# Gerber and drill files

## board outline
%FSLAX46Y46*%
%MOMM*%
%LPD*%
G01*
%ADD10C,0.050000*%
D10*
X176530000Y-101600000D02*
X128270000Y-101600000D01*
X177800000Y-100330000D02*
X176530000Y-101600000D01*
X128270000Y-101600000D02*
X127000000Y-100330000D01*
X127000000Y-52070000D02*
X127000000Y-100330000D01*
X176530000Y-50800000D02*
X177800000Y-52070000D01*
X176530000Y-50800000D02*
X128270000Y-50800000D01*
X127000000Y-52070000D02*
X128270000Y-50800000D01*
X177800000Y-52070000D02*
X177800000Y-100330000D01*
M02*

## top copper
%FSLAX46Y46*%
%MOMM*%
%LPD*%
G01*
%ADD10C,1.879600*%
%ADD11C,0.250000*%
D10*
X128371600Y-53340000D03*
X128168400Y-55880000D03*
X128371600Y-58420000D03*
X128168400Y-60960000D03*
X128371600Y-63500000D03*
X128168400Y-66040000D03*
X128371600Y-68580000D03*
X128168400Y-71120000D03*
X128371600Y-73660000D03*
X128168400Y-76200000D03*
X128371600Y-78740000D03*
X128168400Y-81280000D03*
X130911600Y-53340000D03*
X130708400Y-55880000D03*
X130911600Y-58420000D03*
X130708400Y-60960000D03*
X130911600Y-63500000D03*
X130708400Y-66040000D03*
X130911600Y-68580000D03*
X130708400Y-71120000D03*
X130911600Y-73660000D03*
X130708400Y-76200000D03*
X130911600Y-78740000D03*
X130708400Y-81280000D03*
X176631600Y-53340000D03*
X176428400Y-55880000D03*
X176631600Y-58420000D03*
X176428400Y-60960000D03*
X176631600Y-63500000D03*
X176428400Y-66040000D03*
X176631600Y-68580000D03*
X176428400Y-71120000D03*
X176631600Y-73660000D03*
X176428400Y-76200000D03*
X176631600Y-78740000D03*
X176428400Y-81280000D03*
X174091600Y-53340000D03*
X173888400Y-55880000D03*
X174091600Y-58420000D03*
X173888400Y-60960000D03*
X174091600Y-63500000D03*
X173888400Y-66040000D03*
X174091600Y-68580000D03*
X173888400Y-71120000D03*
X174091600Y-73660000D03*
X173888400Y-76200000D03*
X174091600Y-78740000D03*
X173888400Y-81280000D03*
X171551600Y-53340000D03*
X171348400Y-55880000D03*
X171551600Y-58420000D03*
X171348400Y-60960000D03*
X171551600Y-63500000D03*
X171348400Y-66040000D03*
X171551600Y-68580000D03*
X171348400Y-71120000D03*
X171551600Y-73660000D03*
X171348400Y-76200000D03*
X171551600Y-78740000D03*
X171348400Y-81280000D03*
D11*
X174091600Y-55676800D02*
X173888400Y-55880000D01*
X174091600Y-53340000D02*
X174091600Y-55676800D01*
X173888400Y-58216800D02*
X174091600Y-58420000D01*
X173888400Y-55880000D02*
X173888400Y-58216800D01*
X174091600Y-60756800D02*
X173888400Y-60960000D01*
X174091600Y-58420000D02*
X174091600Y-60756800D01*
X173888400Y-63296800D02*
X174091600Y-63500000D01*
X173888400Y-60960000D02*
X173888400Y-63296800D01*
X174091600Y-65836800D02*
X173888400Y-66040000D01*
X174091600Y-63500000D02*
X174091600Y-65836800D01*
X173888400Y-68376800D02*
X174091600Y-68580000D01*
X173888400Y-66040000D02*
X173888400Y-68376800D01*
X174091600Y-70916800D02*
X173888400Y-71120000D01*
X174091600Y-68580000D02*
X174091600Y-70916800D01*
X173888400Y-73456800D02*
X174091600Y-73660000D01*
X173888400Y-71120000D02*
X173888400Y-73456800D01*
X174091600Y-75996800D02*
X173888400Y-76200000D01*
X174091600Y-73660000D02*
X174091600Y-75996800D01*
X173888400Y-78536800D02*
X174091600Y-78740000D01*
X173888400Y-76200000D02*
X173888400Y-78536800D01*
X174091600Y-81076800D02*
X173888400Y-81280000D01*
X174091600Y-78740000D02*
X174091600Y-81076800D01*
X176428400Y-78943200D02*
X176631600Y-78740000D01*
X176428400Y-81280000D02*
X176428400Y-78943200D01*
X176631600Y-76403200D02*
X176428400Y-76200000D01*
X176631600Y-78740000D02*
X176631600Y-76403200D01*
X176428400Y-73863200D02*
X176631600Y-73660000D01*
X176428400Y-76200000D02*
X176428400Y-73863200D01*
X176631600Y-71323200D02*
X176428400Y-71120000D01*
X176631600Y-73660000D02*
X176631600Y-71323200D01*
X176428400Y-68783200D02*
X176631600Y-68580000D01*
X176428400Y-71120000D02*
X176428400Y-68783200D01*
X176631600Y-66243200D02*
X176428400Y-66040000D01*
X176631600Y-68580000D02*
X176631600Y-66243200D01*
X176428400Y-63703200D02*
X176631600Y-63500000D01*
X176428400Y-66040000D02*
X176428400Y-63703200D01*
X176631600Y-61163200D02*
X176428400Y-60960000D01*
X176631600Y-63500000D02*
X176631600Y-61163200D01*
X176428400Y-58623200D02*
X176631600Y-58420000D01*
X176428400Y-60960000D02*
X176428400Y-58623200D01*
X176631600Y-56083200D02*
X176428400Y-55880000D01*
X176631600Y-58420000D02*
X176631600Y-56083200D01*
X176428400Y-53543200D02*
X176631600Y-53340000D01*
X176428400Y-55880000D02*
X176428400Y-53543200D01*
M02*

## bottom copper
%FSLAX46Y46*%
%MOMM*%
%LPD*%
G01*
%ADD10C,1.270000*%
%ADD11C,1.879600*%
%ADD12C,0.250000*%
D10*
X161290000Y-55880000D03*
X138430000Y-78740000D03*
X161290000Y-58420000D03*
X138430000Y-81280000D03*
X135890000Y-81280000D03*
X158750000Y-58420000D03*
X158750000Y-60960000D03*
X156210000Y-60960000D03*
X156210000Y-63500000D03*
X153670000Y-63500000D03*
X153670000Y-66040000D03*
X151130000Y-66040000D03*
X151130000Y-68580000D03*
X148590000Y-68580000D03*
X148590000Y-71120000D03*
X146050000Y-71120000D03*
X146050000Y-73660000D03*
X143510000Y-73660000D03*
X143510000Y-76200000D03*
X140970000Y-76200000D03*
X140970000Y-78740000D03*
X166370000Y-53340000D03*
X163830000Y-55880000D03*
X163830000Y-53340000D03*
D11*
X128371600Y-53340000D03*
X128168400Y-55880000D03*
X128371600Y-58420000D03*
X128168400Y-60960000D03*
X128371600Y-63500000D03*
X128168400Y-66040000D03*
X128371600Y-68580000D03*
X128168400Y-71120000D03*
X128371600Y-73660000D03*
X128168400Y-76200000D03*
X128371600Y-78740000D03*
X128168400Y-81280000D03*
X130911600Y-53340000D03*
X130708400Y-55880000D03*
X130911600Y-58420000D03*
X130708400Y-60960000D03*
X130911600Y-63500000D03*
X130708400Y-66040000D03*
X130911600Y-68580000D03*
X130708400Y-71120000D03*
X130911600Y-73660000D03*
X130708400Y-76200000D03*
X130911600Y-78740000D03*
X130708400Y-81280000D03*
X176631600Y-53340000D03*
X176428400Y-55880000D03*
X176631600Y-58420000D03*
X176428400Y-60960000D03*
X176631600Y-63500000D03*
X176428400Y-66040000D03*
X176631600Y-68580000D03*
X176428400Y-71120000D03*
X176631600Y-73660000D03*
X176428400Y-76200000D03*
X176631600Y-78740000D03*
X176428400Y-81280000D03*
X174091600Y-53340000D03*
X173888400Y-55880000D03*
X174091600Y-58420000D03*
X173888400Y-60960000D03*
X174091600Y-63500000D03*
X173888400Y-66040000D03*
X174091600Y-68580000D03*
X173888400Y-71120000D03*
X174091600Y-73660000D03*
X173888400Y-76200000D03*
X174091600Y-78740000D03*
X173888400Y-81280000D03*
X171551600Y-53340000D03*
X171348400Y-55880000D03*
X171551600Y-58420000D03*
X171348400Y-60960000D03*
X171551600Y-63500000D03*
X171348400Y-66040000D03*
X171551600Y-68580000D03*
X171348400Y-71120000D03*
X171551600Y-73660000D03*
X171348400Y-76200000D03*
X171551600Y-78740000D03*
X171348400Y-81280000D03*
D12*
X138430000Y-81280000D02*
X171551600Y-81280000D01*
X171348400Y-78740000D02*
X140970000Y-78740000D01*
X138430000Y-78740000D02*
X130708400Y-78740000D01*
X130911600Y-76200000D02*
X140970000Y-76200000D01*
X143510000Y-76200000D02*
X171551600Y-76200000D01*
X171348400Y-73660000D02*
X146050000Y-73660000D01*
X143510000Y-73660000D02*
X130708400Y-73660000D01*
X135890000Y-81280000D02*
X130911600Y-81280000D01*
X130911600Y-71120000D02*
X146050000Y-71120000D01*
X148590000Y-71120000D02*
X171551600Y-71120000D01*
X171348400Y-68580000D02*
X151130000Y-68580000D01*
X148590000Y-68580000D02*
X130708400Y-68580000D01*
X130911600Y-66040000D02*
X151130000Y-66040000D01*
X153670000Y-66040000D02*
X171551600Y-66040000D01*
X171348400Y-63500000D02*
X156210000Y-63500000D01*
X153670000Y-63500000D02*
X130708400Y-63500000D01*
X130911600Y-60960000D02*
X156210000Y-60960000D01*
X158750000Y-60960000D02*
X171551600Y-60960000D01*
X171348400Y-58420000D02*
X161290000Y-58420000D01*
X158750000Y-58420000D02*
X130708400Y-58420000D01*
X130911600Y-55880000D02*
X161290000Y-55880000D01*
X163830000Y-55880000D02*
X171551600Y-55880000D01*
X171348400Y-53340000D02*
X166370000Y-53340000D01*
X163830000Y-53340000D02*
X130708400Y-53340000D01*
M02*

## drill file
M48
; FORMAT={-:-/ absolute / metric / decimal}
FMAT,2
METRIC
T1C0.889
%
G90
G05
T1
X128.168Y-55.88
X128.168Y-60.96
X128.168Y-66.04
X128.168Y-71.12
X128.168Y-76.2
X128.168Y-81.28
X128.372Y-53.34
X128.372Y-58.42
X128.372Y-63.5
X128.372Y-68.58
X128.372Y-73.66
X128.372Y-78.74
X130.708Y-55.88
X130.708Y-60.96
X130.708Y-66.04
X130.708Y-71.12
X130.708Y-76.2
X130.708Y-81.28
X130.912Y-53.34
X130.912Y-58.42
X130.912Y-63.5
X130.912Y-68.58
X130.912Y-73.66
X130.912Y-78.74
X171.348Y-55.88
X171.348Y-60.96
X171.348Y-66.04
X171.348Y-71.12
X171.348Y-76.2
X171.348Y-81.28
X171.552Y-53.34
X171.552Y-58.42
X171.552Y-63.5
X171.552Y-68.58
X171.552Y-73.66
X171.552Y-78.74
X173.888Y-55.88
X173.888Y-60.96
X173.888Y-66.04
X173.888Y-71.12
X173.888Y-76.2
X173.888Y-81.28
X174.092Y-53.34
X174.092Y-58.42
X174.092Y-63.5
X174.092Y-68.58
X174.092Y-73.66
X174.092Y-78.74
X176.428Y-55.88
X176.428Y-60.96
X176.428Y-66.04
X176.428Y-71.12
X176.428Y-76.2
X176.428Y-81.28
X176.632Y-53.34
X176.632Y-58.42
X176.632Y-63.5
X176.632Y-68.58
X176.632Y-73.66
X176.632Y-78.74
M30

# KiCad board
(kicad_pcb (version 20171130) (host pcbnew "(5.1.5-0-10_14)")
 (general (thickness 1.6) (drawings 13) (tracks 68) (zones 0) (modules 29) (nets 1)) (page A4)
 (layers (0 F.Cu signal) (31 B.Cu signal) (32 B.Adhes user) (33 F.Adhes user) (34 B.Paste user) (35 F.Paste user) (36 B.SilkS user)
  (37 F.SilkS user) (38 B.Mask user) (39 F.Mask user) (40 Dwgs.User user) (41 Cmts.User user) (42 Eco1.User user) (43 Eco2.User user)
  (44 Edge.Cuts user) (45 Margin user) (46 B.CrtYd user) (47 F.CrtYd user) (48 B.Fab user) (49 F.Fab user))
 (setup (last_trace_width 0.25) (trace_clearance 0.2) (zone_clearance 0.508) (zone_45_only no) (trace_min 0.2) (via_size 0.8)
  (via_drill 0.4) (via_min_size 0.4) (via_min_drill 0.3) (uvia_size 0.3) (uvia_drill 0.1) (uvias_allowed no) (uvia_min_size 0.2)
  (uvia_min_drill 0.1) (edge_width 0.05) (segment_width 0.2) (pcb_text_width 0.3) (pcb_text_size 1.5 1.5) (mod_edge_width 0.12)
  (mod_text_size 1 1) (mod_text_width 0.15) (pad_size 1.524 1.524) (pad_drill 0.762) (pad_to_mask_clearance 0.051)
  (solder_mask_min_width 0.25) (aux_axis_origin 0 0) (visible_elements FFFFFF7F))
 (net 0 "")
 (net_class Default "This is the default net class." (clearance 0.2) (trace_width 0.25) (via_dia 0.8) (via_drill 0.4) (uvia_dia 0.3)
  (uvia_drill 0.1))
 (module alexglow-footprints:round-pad (layer B.Cu) (at 161.29 55.88)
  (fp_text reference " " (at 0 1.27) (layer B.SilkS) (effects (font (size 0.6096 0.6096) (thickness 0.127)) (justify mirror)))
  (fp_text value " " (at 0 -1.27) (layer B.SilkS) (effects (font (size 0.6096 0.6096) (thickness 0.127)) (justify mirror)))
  (pad P$1 smd circle (at 0 0) (size 1.27 1.27) (layers B.Cu B.Paste B.Mask) (solder_mask_margin 0.1016)))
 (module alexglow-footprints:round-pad (layer B.Cu) (at 138.43 78.74)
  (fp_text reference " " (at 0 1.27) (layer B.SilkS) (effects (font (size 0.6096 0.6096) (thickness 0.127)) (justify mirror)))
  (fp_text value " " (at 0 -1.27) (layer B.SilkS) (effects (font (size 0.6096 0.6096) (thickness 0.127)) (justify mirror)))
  (pad P$1 smd circle (at 0 0) (size 1.27 1.27) (layers B.Cu B.Paste B.Mask) (solder_mask_margin 0.1016)))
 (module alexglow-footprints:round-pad (layer B.Cu) (at 161.29 58.42)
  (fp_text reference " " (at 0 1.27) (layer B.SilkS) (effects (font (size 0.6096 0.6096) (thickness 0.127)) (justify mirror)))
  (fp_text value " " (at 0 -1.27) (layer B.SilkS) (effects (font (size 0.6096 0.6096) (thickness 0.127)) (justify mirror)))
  (pad P$1 smd circle (at 0 0) (size 1.27 1.27) (layers B.Cu B.Paste B.Mask) (solder_mask_margin 0.1016)))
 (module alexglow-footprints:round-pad (layer B.Cu) (at 138.43 81.28)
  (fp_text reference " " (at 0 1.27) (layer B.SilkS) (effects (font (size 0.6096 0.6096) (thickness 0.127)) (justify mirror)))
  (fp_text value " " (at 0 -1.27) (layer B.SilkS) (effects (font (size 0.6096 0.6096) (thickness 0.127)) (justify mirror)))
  (pad P$1 smd circle (at 0 0) (size 1.27 1.27) (layers B.Cu B.Paste B.Mask) (solder_mask_margin 0.1016)))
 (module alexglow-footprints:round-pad (layer B.Cu) (at 135.89 81.28)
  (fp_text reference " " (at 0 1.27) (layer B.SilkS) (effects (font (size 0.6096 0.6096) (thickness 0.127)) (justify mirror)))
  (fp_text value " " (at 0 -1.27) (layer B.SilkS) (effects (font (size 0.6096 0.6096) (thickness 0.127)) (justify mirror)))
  (pad P$1 smd circle (at 0 0) (size 1.27 1.27) (layers B.Cu B.Paste B.Mask) (solder_mask_margin 0.1016)))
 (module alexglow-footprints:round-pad (layer B.Cu) (at 158.75 58.42)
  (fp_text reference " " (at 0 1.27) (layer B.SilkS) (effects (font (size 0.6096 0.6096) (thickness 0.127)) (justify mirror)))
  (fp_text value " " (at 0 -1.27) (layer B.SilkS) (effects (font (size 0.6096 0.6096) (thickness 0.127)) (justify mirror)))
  (pad P$1 smd circle (at 0 0) (size 1.27 1.27) (layers B.Cu B.Paste B.Mask) (solder_mask_margin 0.1016)))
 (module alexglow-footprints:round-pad (layer B.Cu) (at 158.75 60.96)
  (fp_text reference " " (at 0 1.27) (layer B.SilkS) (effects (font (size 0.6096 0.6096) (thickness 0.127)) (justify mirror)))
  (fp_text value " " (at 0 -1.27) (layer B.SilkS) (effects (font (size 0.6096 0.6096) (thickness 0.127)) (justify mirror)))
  (pad P$1 smd circle (at 0 0) (size 1.27 1.27) (layers B.Cu B.Paste B.Mask) (solder_mask_margin 0.1016)))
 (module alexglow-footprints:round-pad (layer B.Cu) (at 156.21 60.96)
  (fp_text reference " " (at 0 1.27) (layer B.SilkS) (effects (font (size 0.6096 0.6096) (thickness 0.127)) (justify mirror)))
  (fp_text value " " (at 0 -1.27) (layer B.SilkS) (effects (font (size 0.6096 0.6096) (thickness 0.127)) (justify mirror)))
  (pad P$1 smd circle (at 0 0) (size 1.27 1.27) (layers B.Cu B.Paste B.Mask) (solder_mask_margin 0.1016)))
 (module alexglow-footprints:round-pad (layer B.Cu) (at 156.21 63.5)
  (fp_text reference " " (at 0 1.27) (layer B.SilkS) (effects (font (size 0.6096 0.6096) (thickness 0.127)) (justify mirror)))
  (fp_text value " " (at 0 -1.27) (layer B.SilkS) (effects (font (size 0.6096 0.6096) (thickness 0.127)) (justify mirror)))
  (pad P$1 smd circle (at 0 0) (size 1.27 1.27) (layers B.Cu B.Paste B.Mask) (solder_mask_margin 0.1016)))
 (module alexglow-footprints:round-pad (layer B.Cu) (at 153.67 63.5)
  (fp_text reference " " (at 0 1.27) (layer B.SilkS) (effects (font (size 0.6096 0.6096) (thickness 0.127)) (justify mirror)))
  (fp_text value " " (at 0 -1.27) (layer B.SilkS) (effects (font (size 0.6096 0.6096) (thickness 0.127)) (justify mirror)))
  (pad P$1 smd circle (at 0 0) (size 1.27 1.27) (layers B.Cu B.Paste B.Mask) (solder_mask_margin 0.1016)))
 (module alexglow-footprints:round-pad (layer B.Cu) (at 153.67 66.04)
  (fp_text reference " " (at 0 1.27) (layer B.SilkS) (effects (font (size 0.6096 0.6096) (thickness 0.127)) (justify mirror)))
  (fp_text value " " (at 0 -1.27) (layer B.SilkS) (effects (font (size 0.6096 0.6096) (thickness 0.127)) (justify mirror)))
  (pad P$1 smd circle (at 0 0) (size 1.27 1.27) (layers B.Cu B.Paste B.Mask) (solder_mask_margin 0.1016)))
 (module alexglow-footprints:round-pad (layer B.Cu) (at 151.13 66.04)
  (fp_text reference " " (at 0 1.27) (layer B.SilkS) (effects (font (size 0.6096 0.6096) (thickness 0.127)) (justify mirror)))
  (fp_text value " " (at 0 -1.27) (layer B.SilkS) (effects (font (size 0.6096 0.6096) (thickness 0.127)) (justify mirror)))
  (pad P$1 smd circle (at 0 0) (size 1.27 1.27) (layers B.Cu B.Paste B.Mask) (solder_mask_margin 0.1016)))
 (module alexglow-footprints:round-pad (layer B.Cu) (at 151.13 68.58)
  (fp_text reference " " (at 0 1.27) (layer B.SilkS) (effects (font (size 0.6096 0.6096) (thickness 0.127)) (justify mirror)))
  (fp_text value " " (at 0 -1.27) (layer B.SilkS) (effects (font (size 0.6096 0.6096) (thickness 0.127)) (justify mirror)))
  (pad P$1 smd circle (at 0 0) (size 1.27 1.27) (layers B.Cu B.Paste B.Mask) (solder_mask_margin 0.1016)))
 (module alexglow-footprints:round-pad (layer B.Cu) (at 148.59 68.58)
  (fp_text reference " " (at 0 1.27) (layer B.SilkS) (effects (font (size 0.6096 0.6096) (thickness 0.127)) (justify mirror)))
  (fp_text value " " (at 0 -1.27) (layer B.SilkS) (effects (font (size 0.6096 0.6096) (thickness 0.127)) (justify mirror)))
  (pad P$1 smd circle (at 0 0) (size 1.27 1.27) (layers B.Cu B.Paste B.Mask) (solder_mask_margin 0.1016)))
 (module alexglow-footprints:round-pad (layer B.Cu) (at 148.59 71.12)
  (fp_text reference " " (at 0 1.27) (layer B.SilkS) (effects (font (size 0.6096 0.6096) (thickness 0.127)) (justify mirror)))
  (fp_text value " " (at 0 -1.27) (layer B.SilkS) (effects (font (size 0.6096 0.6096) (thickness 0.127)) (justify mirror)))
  (pad P$1 smd circle (at 0 0) (size 1.27 1.27) (layers B.Cu B.Paste B.Mask) (solder_mask_margin 0.1016)))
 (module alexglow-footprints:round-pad (layer B.Cu) (at 146.05 71.12)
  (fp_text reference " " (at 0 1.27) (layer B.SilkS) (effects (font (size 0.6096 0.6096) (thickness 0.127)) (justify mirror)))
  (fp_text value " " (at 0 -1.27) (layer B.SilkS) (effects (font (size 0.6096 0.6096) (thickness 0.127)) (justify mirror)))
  (pad P$1 smd circle (at 0 0) (size 1.27 1.27) (layers B.Cu B.Paste B.Mask) (solder_mask_margin 0.1016)))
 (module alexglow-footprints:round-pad (layer B.Cu) (at 146.05 73.66)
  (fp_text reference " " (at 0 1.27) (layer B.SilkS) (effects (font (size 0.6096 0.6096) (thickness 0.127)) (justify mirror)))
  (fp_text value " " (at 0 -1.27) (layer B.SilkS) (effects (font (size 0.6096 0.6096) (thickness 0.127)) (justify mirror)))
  (pad P$1 smd circle (at 0 0) (size 1.27 1.27) (layers B.Cu B.Paste B.Mask) (solder_mask_margin 0.1016)))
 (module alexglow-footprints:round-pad (layer B.Cu) (at 143.51 73.66)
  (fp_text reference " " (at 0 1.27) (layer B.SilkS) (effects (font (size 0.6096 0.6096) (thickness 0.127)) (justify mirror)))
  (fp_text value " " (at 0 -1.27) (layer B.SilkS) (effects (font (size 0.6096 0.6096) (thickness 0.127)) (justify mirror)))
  (pad P$1 smd circle (at 0 0) (size 1.27 1.27) (layers B.Cu B.Paste B.Mask) (solder_mask_margin 0.1016)))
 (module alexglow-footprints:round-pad (layer B.Cu) (at 143.51 76.2)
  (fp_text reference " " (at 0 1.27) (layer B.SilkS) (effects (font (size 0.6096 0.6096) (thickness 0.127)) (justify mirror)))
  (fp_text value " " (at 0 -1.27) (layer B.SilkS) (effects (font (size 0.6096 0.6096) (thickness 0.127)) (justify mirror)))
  (pad P$1 smd circle (at 0 0) (size 1.27 1.27) (layers B.Cu B.Paste B.Mask) (solder_mask_margin 0.1016)))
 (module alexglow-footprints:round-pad (layer B.Cu) (at 140.97 76.2)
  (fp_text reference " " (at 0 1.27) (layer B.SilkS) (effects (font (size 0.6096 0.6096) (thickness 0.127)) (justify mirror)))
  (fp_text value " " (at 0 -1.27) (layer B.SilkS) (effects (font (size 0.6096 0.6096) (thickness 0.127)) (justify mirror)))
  (pad P$1 smd circle (at 0 0) (size 1.27 1.27) (layers B.Cu B.Paste B.Mask) (solder_mask_margin 0.1016)))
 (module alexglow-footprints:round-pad (layer B.Cu) (at 140.97 78.74)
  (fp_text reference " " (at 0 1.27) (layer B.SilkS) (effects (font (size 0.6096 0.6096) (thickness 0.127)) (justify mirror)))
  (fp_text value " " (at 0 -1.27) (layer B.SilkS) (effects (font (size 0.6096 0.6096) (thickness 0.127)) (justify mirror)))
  (pad P$1 smd circle (at 0 0) (size 1.27 1.27) (layers B.Cu B.Paste B.Mask) (solder_mask_margin 0.1016)))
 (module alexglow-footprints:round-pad (layer B.Cu) (at 166.37 53.34)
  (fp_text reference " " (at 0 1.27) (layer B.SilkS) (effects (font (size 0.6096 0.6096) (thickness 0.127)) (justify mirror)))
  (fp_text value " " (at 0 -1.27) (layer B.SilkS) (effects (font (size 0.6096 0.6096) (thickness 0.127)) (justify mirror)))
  (pad P$1 smd circle (at 0 0) (size 1.27 1.27) (layers B.Cu B.Paste B.Mask) (solder_mask_margin 0.1016)))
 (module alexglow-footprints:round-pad (layer B.Cu) (at 163.83 55.88)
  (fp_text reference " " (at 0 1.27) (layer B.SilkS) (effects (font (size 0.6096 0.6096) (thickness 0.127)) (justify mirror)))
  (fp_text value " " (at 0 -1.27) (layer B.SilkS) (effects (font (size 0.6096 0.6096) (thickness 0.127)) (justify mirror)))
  (pad P$1 smd circle (at 0 0) (size 1.27 1.27) (layers B.Cu B.Paste B.Mask) (solder_mask_margin 0.1016)))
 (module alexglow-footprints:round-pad (layer B.Cu) (at 163.83 53.34)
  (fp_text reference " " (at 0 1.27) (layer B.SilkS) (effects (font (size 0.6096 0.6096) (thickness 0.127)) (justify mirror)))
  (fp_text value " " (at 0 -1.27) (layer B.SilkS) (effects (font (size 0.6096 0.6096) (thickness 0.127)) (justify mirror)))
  (pad P$1 smd circle (at 0 0) (size 1.27 1.27) (layers B.Cu B.Paste B.Mask) (solder_mask_margin 0.1016)))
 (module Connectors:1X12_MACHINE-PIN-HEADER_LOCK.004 (layer F.Cu) (at 128.27 81.28 90)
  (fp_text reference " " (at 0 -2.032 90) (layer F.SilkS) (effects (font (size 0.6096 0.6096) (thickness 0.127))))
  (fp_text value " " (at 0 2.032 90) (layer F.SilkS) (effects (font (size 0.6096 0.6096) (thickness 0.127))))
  (pad 12 thru_hole circle (at 27.94 0.1016 90) (size 1.8796 1.8796) (drill 0.889) (layers *.Cu *.Mask) (solder_mask_margin 0.1016))
  (pad 11 thru_hole circle (at 25.4 -0.1016 90) (size 1.8796 1.8796) (drill 0.889) (layers *.Cu *.Mask) (solder_mask_margin 0.1016))
  (pad 10 thru_hole circle (at 22.86 0.1016 90) (size 1.8796 1.8796) (drill 0.889) (layers *.Cu *.Mask) (solder_mask_margin 0.1016))
  (pad 9 thru_hole circle (at 20.32 -0.1016 90) (size 1.8796 1.8796) (drill 0.889) (layers *.Cu *.Mask) (solder_mask_margin 0.1016))
  (pad 8 thru_hole circle (at 17.78 0.1016 90) (size 1.8796 1.8796) (drill 0.889) (layers *.Cu *.Mask) (solder_mask_margin 0.1016))
  (pad 7 thru_hole circle (at 15.24 -0.1016 90) (size 1.8796 1.8796) (drill 0.889) (layers *.Cu *.Mask) (solder_mask_margin 0.1016))
  (pad 6 thru_hole circle (at 12.7 0.1016 90) (size 1.8796 1.8796) (drill 0.889) (layers *.Cu *.Mask) (solder_mask_margin 0.1016))
  (pad 5 thru_hole circle (at 10.16 -0.1016 90) (size 1.8796 1.8796) (drill 0.889) (layers *.Cu *.Mask) (solder_mask_margin 0.1016))
  (pad 4 thru_hole circle (at 7.62 0.1016 90) (size 1.8796 1.8796) (drill 0.889) (layers *.Cu *.Mask) (solder_mask_margin 0.1016))
  (pad 3 thru_hole circle (at 5.08 -0.1016 90) (size 1.8796 1.8796) (drill 0.889) (layers *.Cu *.Mask) (solder_mask_margin 0.1016))
  (pad 2 thru_hole circle (at 2.54 0.1016 90) (size 1.8796 1.8796) (drill 0.889) (layers *.Cu *.Mask) (solder_mask_margin 0.1016))
  (pad 1 thru_hole circle (at 0 -0.1016 90) (size 1.8796 1.8796) (drill 0.889) (layers *.Cu *.Mask) (solder_mask_margin 0.1016)))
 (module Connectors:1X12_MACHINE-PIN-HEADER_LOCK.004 (layer F.Cu) (at 130.81 81.28 90)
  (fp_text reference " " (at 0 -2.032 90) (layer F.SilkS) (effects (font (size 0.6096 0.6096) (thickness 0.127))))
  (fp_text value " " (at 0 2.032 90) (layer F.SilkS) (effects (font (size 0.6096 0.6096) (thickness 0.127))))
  (pad 12 thru_hole circle (at 27.94 0.1016 90) (size 1.8796 1.8796) (drill 0.889) (layers *.Cu *.Mask) (solder_mask_margin 0.1016))
  (pad 11 thru_hole circle (at 25.4 -0.1016 90) (size 1.8796 1.8796) (drill 0.889) (layers *.Cu *.Mask) (solder_mask_margin 0.1016))
  (pad 10 thru_hole circle (at 22.86 0.1016 90) (size 1.8796 1.8796) (drill 0.889) (layers *.Cu *.Mask) (solder_mask_margin 0.1016))
  (pad 9 thru_hole circle (at 20.32 -0.1016 90) (size 1.8796 1.8796) (drill 0.889) (layers *.Cu *.Mask) (solder_mask_margin 0.1016))
  (pad 8 thru_hole circle (at 17.78 0.1016 90) (size 1.8796 1.8796) (drill 0.889) (layers *.Cu *.Mask) (solder_mask_margin 0.1016))
  (pad 7 thru_hole circle (at 15.24 -0.1016 90) (size 1.8796 1.8796) (drill 0.889) (layers *.Cu *.Mask) (solder_mask_margin 0.1016))
  (pad 6 thru_hole circle (at 12.7 0.1016 90) (size 1.8796 1.8796) (drill 0.889) (layers *.Cu *.Mask) (solder_mask_margin 0.1016))
  (pad 5 thru_hole circle (at 10.16 -0.1016 90) (size 1.8796 1.8796) (drill 0.889) (layers *.Cu *.Mask) (solder_mask_margin 0.1016))
  (pad 4 thru_hole circle (at 7.62 0.1016 90) (size 1.8796 1.8796) (drill 0.889) (layers *.Cu *.Mask) (solder_mask_margin 0.1016))
  (pad 3 thru_hole circle (at 5.08 -0.1016 90) (size 1.8796 1.8796) (drill 0.889) (layers *.Cu *.Mask) (solder_mask_margin 0.1016))
  (pad 2 thru_hole circle (at 2.54 0.1016 90) (size 1.8796 1.8796) (drill 0.889) (layers *.Cu *.Mask) (solder_mask_margin 0.1016))
  (pad 1 thru_hole circle (at 0 -0.1016 90) (size 1.8796 1.8796) (drill 0.889) (layers *.Cu *.Mask) (solder_mask_margin 0.1016)))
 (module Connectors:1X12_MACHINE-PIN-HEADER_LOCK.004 (layer F.Cu) (at 176.53 81.28 90)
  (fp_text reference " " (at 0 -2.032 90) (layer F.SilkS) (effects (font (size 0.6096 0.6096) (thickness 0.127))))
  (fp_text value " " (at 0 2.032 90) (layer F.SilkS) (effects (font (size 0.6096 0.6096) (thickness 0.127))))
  (pad 12 thru_hole circle (at 27.94 0.1016 90) (size 1.8796 1.8796) (drill 0.889) (layers *.Cu *.Mask) (solder_mask_margin 0.1016))
  (pad 11 thru_hole circle (at 25.4 -0.1016 90) (size 1.8796 1.8796) (drill 0.889) (layers *.Cu *.Mask) (solder_mask_margin 0.1016))
  (pad 10 thru_hole circle (at 22.86 0.1016 90) (size 1.8796 1.8796) (drill 0.889) (layers *.Cu *.Mask) (solder_mask_margin 0.1016))
  (pad 9 thru_hole circle (at 20.32 -0.1016 90) (size 1.8796 1.8796) (drill 0.889) (layers *.Cu *.Mask) (solder_mask_margin 0.1016))
  (pad 8 thru_hole circle (at 17.78 0.1016 90) (size 1.8796 1.8796) (drill 0.889) (layers *.Cu *.Mask) (solder_mask_margin 0.1016))
  (pad 7 thru_hole circle (at 15.24 -0.1016 90) (size 1.8796 1.8796) (drill 0.889) (layers *.Cu *.Mask) (solder_mask_margin 0.1016))
  (pad 6 thru_hole circle (at 12.7 0.1016 90) (size 1.8796 1.8796) (drill 0.889) (layers *.Cu *.Mask) (solder_mask_margin 0.1016))
  (pad 5 thru_hole circle (at 10.16 -0.1016 90) (size 1.8796 1.8796) (drill 0.889) (layers *.Cu *.Mask) (solder_mask_margin 0.1016))
  (pad 4 thru_hole circle (at 7.62 0.1016 90) (size 1.8796 1.8796) (drill 0.889) (layers *.Cu *.Mask) (solder_mask_margin 0.1016))
  (pad 3 thru_hole circle (at 5.08 -0.1016 90) (size 1.8796 1.8796) (drill 0.889) (layers *.Cu *.Mask) (solder_mask_margin 0.1016))
  (pad 2 thru_hole circle (at 2.54 0.1016 90) (size 1.8796 1.8796) (drill 0.889) (layers *.Cu *.Mask) (solder_mask_margin 0.1016))
  (pad 1 thru_hole circle (at 0 -0.1016 90) (size 1.8796 1.8796) (drill 0.889) (layers *.Cu *.Mask) (solder_mask_margin 0.1016)))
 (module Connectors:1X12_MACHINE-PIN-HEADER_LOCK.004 (layer F.Cu) (at 173.99 81.28 90)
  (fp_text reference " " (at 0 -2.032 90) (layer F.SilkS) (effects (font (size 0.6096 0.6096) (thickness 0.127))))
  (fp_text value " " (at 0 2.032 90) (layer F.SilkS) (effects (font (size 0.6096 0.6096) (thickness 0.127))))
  (pad 12 thru_hole circle (at 27.94 0.1016 90) (size 1.8796 1.8796) (drill 0.889) (layers *.Cu *.Mask) (solder_mask_margin 0.1016))
  (pad 11 thru_hole circle (at 25.4 -0.1016 90) (size 1.8796 1.8796) (drill 0.889) (layers *.Cu *.Mask) (solder_mask_margin 0.1016))
  (pad 10 thru_hole circle (at 22.86 0.1016 90) (size 1.8796 1.8796) (drill 0.889) (layers *.Cu *.Mask) (solder_mask_margin 0.1016))
  (pad 9 thru_hole circle (at 20.32 -0.1016 90) (size 1.8796 1.8796) (drill 0.889) (layers *.Cu *.Mask) (solder_mask_margin 0.1016))
  (pad 8 thru_hole circle (at 17.78 0.1016 90) (size 1.8796 1.8796) (drill 0.889) (layers *.Cu *.Mask) (solder_mask_margin 0.1016))
  (pad 7 thru_hole circle (at 15.24 -0.1016 90) (size 1.8796 1.8796) (drill 0.889) (layers *.Cu *.Mask) (solder_mask_margin 0.1016))
  (pad 6 thru_hole circle (at 12.7 0.1016 90) (size 1.8796 1.8796) (drill 0.889) (layers *.Cu *.Mask) (solder_mask_margin 0.1016))
  (pad 5 thru_hole circle (at 10.16 -0.1016 90) (size 1.8796 1.8796) (drill 0.889) (layers *.Cu *.Mask) (solder_mask_margin 0.1016))
  (pad 4 thru_hole circle (at 7.62 0.1016 90) (size 1.8796 1.8796) (drill 0.889) (layers *.Cu *.Mask) (solder_mask_margin 0.1016))
  (pad 3 thru_hole circle (at 5.08 -0.1016 90) (size 1.8796 1.8796) (drill 0.889) (layers *.Cu *.Mask) (solder_mask_margin 0.1016))
  (pad 2 thru_hole circle (at 2.54 0.1016 90) (size 1.8796 1.8796) (drill 0.889) (layers *.Cu *.Mask) (solder_mask_margin 0.1016))
  (pad 1 thru_hole circle (at 0 -0.1016 90) (size 1.8796 1.8796) (drill 0.889) (layers *.Cu *.Mask) (solder_mask_margin 0.1016)))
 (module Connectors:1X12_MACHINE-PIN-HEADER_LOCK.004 (layer F.Cu) (at 171.45 81.28 90)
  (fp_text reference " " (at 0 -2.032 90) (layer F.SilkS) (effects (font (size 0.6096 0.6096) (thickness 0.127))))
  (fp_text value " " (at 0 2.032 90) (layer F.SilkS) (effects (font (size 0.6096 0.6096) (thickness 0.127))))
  (pad 12 thru_hole circle (at 27.94 0.1016 90) (size 1.8796 1.8796) (drill 0.889) (layers *.Cu *.Mask) (solder_mask_margin 0.1016))
  (pad 11 thru_hole circle (at 25.4 -0.1016 90) (size 1.8796 1.8796) (drill 0.889) (layers *.Cu *.Mask) (solder_mask_margin 0.1016))
  (pad 10 thru_hole circle (at 22.86 0.1016 90) (size 1.8796 1.8796) (drill 0.889) (layers *.Cu *.Mask) (solder_mask_margin 0.1016))
  (pad 9 thru_hole circle (at 20.32 -0.1016 90) (size 1.8796 1.8796) (drill 0.889) (layers *.Cu *.Mask) (solder_mask_margin 0.1016))
  (pad 8 thru_hole circle (at 17.78 0.1016 90) (size 1.8796 1.8796) (drill 0.889) (layers *.Cu *.Mask) (solder_mask_margin 0.1016))
  (pad 7 thru_hole circle (at 15.24 -0.1016 90) (size 1.8796 1.8796) (drill 0.889) (layers *.Cu *.Mask) (solder_mask_margin 0.1016))
  (pad 6 thru_hole circle (at 12.7 0.1016 90) (size 1.8796 1.8796) (drill 0.889) (layers *.Cu *.Mask) (solder_mask_margin 0.1016))
  (pad 5 thru_hole circle (at 10.16 -0.1016 90) (size 1.8796 1.8796) (drill 0.889) (layers *.Cu *.Mask) (solder_mask_margin 0.1016))
  (pad 4 thru_hole circle (at 7.62 0.1016 90) (size 1.8796 1.8796) (drill 0.889) (layers *.Cu *.Mask) (solder_mask_margin 0.1016))
  (pad 3 thru_hole circle (at 5.08 -0.1016 90) (size 1.8796 1.8796) (drill 0.889) (layers *.Cu *.Mask) (solder_mask_margin 0.1016))
  (pad 2 thru_hole circle (at 2.54 0.1016 90) (size 1.8796 1.8796) (drill 0.889) (layers *.Cu *.Mask) (solder_mask_margin 0.1016))
  (pad 1 thru_hole circle (at 0 -0.1016 90) (size 1.8796 1.8796) (drill 0.889) (layers *.Cu *.Mask) (solder_mask_margin 0.1016)))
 (gr_line (start 176.53 101.6) (end 128.27 101.6) (layer Edge.Cuts) (width 0.05))
 (gr_line (start 177.8 100.33) (end 176.53 101.6) (layer Edge.Cuts) (width 0.05))
 (gr_line (start 128.27 101.6) (end 127 100.33) (layer Edge.Cuts) (width 0.05))
 (gr_line (start 127 52.07) (end 127 100.33) (layer Edge.Cuts) (width 0.05))
 (gr_line (start 176.53 50.8) (end 177.8 52.07) (layer Edge.Cuts) (width 0.05))
 (gr_line (start 176.53 50.8) (end 128.27 50.8) (layer Edge.Cuts) (width 0.05))
 (gr_line (start 127 52.07) (end 128.27 50.8) (layer Edge.Cuts) (width 0.05))
 (gr_line (start 177.8 52.07) (end 177.8 100.33) (layer Edge.Cuts) (width 0.05))
 (segment (start 174.0916 55.6768) (end 173.8884 55.88) (width 0.25) (layer F.Cu) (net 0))
 (segment (start 174.0916 53.34) (end 174.0916 55.6768) (width 0.25) (layer F.Cu) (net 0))
 (segment (start 173.8884 58.2168) (end 174.0916 58.42) (width 0.25) (layer F.Cu) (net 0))
 (segment (start 173.8884 55.88) (end 173.8884 58.2168) (width 0.25) (layer F.Cu) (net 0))
 (segment (start 174.0916 60.7568) (end 173.8884 60.96) (width 0.25) (layer F.Cu) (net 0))
 (segment (start 174.0916 58.42) (end 174.0916 60.7568) (width 0.25) (layer F.Cu) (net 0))
 (segment (start 173.8884 63.2968) (end 174.0916 63.5) (width 0.25) (layer F.Cu) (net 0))
 (segment (start 173.8884 60.96) (end 173.8884 63.2968) (width 0.25) (layer F.Cu) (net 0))
 (segment (start 174.0916 65.8368) (end 173.8884 66.04) (width 0.25) (layer F.Cu) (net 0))
 (segment (start 174.0916 63.5) (end 174.0916 65.8368) (width 0.25) (layer F.Cu) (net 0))
 (segment (start 173.8884 68.3768) (end 174.0916 68.58) (width 0.25) (layer F.Cu) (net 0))
 (segment (start 173.8884 66.04) (end 173.8884 68.3768) (width 0.25) (layer F.Cu) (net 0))
 (segment (start 174.0916 70.9168) (end 173.8884 71.12) (width 0.25) (layer F.Cu) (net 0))
 (segment (start 174.0916 68.58) (end 174.0916 70.9168) (width 0.25) (layer F.Cu) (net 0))
 (segment (start 173.8884 73.4568) (end 174.0916 73.66) (width 0.25) (layer F.Cu) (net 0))
 (segment (start 173.8884 71.12) (end 173.8884 73.4568) (width 0.25) (layer F.Cu) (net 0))
 (segment (start 174.0916 75.9968) (end 173.8884 76.2) (width 0.25) (layer F.Cu) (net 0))
 (segment (start 174.0916 73.66) (end 174.0916 75.9968) (width 0.25) (layer F.Cu) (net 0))
 (segment (start 173.8884 78.5368) (end 174.0916 78.74) (width 0.25) (layer F.Cu) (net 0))
 (segment (start 173.8884 76.2) (end 173.8884 78.5368) (width 0.25) (layer F.Cu) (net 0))
 (segment (start 174.0916 81.0768) (end 173.8884 81.28) (width 0.25) (layer F.Cu) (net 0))
 (segment (start 174.0916 78.74) (end 174.0916 81.0768) (width 0.25) (layer F.Cu) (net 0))
 (segment (start 176.4284 78.9432) (end 176.6316 78.74) (width 0.25) (layer F.Cu) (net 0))
 (segment (start 176.4284 81.28) (end 176.4284 78.9432) (width 0.25) (layer F.Cu) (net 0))
 (segment (start 176.6316 76.4032) (end 176.4284 76.2) (width 0.25) (layer F.Cu) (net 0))
 (segment (start 176.6316 78.74) (end 176.6316 76.4032) (width 0.25) (layer F.Cu) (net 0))
 (segment (start 176.4284 73.8632) (end 176.6316 73.66) (width 0.25) (layer F.Cu) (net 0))
 (segment (start 176.4284 76.2) (end 176.4284 73.8632) (width 0.25) (layer F.Cu) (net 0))
 (segment (start 176.6316 71.3232) (end 176.4284 71.12) (width 0.25) (layer F.Cu) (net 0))
 (segment (start 176.6316 73.66) (end 176.6316 71.3232) (width 0.25) (layer F.Cu) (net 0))
 (segment (start 176.4284 68.7832) (end 176.6316 68.58) (width 0.25) (layer F.Cu) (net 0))
 (segment (start 176.4284 71.12) (end 176.4284 68.7832) (width 0.25) (layer F.Cu) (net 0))
 (segment (start 176.6316 66.2432) (end 176.4284 66.04) (width 0.25) (layer F.Cu) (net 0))
 (segment (start 176.6316 68.58) (end 176.6316 66.2432) (width 0.25) (layer F.Cu) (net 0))
 (segment (start 176.4284 63.7032) (end 176.6316 63.5) (width 0.25) (layer F.Cu) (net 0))
 (segment (start 176.4284 66.04) (end 176.4284 63.7032) (width 0.25) (layer F.Cu) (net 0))
 (segment (start 176.6316 61.1632) (end 176.4284 60.96) (width 0.25) (layer F.Cu) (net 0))
 (segment (start 176.6316 63.5) (end 176.6316 61.1632) (width 0.25) (layer F.Cu) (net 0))
 (segment (start 176.4284 58.6232) (end 176.6316 58.42) (width 0.25) (layer F.Cu) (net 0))
 (segment (start 176.4284 60.96) (end 176.4284 58.6232) (width 0.25) (layer F.Cu) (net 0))
 (segment (start 176.6316 56.0832) (end 176.4284 55.88) (width 0.25) (layer F.Cu) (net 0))
 (segment (start 176.6316 58.42) (end 176.6316 56.0832) (width 0.25) (layer F.Cu) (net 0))
 (segment (start 176.4284 53.5432) (end 176.6316 53.34) (width 0.25) (layer F.Cu) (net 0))
 (segment (start 176.4284 55.88) (end 176.4284 53.5432) (width 0.25) (layer F.Cu) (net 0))
 (segment (start 138.43 81.28) (end 171.5516 81.28) (width 0.25) (layer B.Cu) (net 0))
 (segment (start 171.3484 78.74) (end 140.97 78.74) (width 0.25) (layer B.Cu) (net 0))
 (segment (start 138.43 78.74) (end 130.7084 78.74) (width 0.25) (layer B.Cu) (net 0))
 (segment (start 130.9116 76.2) (end 140.97 76.2) (width 0.25) (layer B.Cu) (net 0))
 (segment (start 143.51 76.2) (end 171.5516 76.2) (width 0.25) (layer B.Cu) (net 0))
 (segment (start 171.3484 73.66) (end 146.05 73.66) (width 0.25) (layer B.Cu) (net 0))
 (segment (start 143.51 73.66) (end 130.7084 73.66) (width 0.25) (layer B.Cu) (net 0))
 (segment (start 135.89 81.28) (end 130.9116 81.28) (width 0.25) (layer B.Cu) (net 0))
 (segment (start 130.9116 71.12) (end 146.05 71.12) (width 0.25) (layer B.Cu) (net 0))
 (segment (start 148.59 71.12) (end 171.5516 71.12) (width 0.25) (layer B.Cu) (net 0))
 (segment (start 171.3484 68.58) (end 151.13 68.58) (width 0.25) (layer B.Cu) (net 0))
 (segment (start 148.59 68.58) (end 130.7084 68.58) (width 0.25) (layer B.Cu) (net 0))
 (segment (start 130.9116 66.04) (end 151.13 66.04) (width 0.25) (layer B.Cu) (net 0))
 (segment (start 153.67 66.04) (end 171.5516 66.04) (width 0.25) (layer B.Cu) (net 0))
 (segment (start 171.3484 63.5) (end 156.21 63.5) (width 0.25) (layer B.Cu) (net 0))
 (segment (start 153.67 63.5) (end 130.7084 63.5) (width 0.25) (layer B.Cu) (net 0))
 (segment (start 130.9116 60.96) (end 156.21 60.96) (width 0.25) (layer B.Cu) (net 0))
 (segment (start 158.75 60.96) (end 171.5516 60.96) (width 0.25) (layer B.Cu) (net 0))
 (segment (start 171.3484 58.42) (end 161.29 58.42) (width 0.25) (layer B.Cu) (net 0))
 (segment (start 158.75 58.42) (end 130.7084 58.42) (width 0.25) (layer B.Cu) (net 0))
 (segment (start 130.9116 55.88) (end 161.29 55.88) (width 0.25) (layer B.Cu) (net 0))
 (segment (start 163.83 55.88) (end 171.5516 55.88) (width 0.25) (layer B.Cu) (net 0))
 (segment (start 171.3484 53.34) (end 166.37 53.34) (width 0.25) (layer B.Cu) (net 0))
 (segment (start 163.83 53.34) (end 130.7084 53.34) (width 0.25) (layer B.Cu) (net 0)))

